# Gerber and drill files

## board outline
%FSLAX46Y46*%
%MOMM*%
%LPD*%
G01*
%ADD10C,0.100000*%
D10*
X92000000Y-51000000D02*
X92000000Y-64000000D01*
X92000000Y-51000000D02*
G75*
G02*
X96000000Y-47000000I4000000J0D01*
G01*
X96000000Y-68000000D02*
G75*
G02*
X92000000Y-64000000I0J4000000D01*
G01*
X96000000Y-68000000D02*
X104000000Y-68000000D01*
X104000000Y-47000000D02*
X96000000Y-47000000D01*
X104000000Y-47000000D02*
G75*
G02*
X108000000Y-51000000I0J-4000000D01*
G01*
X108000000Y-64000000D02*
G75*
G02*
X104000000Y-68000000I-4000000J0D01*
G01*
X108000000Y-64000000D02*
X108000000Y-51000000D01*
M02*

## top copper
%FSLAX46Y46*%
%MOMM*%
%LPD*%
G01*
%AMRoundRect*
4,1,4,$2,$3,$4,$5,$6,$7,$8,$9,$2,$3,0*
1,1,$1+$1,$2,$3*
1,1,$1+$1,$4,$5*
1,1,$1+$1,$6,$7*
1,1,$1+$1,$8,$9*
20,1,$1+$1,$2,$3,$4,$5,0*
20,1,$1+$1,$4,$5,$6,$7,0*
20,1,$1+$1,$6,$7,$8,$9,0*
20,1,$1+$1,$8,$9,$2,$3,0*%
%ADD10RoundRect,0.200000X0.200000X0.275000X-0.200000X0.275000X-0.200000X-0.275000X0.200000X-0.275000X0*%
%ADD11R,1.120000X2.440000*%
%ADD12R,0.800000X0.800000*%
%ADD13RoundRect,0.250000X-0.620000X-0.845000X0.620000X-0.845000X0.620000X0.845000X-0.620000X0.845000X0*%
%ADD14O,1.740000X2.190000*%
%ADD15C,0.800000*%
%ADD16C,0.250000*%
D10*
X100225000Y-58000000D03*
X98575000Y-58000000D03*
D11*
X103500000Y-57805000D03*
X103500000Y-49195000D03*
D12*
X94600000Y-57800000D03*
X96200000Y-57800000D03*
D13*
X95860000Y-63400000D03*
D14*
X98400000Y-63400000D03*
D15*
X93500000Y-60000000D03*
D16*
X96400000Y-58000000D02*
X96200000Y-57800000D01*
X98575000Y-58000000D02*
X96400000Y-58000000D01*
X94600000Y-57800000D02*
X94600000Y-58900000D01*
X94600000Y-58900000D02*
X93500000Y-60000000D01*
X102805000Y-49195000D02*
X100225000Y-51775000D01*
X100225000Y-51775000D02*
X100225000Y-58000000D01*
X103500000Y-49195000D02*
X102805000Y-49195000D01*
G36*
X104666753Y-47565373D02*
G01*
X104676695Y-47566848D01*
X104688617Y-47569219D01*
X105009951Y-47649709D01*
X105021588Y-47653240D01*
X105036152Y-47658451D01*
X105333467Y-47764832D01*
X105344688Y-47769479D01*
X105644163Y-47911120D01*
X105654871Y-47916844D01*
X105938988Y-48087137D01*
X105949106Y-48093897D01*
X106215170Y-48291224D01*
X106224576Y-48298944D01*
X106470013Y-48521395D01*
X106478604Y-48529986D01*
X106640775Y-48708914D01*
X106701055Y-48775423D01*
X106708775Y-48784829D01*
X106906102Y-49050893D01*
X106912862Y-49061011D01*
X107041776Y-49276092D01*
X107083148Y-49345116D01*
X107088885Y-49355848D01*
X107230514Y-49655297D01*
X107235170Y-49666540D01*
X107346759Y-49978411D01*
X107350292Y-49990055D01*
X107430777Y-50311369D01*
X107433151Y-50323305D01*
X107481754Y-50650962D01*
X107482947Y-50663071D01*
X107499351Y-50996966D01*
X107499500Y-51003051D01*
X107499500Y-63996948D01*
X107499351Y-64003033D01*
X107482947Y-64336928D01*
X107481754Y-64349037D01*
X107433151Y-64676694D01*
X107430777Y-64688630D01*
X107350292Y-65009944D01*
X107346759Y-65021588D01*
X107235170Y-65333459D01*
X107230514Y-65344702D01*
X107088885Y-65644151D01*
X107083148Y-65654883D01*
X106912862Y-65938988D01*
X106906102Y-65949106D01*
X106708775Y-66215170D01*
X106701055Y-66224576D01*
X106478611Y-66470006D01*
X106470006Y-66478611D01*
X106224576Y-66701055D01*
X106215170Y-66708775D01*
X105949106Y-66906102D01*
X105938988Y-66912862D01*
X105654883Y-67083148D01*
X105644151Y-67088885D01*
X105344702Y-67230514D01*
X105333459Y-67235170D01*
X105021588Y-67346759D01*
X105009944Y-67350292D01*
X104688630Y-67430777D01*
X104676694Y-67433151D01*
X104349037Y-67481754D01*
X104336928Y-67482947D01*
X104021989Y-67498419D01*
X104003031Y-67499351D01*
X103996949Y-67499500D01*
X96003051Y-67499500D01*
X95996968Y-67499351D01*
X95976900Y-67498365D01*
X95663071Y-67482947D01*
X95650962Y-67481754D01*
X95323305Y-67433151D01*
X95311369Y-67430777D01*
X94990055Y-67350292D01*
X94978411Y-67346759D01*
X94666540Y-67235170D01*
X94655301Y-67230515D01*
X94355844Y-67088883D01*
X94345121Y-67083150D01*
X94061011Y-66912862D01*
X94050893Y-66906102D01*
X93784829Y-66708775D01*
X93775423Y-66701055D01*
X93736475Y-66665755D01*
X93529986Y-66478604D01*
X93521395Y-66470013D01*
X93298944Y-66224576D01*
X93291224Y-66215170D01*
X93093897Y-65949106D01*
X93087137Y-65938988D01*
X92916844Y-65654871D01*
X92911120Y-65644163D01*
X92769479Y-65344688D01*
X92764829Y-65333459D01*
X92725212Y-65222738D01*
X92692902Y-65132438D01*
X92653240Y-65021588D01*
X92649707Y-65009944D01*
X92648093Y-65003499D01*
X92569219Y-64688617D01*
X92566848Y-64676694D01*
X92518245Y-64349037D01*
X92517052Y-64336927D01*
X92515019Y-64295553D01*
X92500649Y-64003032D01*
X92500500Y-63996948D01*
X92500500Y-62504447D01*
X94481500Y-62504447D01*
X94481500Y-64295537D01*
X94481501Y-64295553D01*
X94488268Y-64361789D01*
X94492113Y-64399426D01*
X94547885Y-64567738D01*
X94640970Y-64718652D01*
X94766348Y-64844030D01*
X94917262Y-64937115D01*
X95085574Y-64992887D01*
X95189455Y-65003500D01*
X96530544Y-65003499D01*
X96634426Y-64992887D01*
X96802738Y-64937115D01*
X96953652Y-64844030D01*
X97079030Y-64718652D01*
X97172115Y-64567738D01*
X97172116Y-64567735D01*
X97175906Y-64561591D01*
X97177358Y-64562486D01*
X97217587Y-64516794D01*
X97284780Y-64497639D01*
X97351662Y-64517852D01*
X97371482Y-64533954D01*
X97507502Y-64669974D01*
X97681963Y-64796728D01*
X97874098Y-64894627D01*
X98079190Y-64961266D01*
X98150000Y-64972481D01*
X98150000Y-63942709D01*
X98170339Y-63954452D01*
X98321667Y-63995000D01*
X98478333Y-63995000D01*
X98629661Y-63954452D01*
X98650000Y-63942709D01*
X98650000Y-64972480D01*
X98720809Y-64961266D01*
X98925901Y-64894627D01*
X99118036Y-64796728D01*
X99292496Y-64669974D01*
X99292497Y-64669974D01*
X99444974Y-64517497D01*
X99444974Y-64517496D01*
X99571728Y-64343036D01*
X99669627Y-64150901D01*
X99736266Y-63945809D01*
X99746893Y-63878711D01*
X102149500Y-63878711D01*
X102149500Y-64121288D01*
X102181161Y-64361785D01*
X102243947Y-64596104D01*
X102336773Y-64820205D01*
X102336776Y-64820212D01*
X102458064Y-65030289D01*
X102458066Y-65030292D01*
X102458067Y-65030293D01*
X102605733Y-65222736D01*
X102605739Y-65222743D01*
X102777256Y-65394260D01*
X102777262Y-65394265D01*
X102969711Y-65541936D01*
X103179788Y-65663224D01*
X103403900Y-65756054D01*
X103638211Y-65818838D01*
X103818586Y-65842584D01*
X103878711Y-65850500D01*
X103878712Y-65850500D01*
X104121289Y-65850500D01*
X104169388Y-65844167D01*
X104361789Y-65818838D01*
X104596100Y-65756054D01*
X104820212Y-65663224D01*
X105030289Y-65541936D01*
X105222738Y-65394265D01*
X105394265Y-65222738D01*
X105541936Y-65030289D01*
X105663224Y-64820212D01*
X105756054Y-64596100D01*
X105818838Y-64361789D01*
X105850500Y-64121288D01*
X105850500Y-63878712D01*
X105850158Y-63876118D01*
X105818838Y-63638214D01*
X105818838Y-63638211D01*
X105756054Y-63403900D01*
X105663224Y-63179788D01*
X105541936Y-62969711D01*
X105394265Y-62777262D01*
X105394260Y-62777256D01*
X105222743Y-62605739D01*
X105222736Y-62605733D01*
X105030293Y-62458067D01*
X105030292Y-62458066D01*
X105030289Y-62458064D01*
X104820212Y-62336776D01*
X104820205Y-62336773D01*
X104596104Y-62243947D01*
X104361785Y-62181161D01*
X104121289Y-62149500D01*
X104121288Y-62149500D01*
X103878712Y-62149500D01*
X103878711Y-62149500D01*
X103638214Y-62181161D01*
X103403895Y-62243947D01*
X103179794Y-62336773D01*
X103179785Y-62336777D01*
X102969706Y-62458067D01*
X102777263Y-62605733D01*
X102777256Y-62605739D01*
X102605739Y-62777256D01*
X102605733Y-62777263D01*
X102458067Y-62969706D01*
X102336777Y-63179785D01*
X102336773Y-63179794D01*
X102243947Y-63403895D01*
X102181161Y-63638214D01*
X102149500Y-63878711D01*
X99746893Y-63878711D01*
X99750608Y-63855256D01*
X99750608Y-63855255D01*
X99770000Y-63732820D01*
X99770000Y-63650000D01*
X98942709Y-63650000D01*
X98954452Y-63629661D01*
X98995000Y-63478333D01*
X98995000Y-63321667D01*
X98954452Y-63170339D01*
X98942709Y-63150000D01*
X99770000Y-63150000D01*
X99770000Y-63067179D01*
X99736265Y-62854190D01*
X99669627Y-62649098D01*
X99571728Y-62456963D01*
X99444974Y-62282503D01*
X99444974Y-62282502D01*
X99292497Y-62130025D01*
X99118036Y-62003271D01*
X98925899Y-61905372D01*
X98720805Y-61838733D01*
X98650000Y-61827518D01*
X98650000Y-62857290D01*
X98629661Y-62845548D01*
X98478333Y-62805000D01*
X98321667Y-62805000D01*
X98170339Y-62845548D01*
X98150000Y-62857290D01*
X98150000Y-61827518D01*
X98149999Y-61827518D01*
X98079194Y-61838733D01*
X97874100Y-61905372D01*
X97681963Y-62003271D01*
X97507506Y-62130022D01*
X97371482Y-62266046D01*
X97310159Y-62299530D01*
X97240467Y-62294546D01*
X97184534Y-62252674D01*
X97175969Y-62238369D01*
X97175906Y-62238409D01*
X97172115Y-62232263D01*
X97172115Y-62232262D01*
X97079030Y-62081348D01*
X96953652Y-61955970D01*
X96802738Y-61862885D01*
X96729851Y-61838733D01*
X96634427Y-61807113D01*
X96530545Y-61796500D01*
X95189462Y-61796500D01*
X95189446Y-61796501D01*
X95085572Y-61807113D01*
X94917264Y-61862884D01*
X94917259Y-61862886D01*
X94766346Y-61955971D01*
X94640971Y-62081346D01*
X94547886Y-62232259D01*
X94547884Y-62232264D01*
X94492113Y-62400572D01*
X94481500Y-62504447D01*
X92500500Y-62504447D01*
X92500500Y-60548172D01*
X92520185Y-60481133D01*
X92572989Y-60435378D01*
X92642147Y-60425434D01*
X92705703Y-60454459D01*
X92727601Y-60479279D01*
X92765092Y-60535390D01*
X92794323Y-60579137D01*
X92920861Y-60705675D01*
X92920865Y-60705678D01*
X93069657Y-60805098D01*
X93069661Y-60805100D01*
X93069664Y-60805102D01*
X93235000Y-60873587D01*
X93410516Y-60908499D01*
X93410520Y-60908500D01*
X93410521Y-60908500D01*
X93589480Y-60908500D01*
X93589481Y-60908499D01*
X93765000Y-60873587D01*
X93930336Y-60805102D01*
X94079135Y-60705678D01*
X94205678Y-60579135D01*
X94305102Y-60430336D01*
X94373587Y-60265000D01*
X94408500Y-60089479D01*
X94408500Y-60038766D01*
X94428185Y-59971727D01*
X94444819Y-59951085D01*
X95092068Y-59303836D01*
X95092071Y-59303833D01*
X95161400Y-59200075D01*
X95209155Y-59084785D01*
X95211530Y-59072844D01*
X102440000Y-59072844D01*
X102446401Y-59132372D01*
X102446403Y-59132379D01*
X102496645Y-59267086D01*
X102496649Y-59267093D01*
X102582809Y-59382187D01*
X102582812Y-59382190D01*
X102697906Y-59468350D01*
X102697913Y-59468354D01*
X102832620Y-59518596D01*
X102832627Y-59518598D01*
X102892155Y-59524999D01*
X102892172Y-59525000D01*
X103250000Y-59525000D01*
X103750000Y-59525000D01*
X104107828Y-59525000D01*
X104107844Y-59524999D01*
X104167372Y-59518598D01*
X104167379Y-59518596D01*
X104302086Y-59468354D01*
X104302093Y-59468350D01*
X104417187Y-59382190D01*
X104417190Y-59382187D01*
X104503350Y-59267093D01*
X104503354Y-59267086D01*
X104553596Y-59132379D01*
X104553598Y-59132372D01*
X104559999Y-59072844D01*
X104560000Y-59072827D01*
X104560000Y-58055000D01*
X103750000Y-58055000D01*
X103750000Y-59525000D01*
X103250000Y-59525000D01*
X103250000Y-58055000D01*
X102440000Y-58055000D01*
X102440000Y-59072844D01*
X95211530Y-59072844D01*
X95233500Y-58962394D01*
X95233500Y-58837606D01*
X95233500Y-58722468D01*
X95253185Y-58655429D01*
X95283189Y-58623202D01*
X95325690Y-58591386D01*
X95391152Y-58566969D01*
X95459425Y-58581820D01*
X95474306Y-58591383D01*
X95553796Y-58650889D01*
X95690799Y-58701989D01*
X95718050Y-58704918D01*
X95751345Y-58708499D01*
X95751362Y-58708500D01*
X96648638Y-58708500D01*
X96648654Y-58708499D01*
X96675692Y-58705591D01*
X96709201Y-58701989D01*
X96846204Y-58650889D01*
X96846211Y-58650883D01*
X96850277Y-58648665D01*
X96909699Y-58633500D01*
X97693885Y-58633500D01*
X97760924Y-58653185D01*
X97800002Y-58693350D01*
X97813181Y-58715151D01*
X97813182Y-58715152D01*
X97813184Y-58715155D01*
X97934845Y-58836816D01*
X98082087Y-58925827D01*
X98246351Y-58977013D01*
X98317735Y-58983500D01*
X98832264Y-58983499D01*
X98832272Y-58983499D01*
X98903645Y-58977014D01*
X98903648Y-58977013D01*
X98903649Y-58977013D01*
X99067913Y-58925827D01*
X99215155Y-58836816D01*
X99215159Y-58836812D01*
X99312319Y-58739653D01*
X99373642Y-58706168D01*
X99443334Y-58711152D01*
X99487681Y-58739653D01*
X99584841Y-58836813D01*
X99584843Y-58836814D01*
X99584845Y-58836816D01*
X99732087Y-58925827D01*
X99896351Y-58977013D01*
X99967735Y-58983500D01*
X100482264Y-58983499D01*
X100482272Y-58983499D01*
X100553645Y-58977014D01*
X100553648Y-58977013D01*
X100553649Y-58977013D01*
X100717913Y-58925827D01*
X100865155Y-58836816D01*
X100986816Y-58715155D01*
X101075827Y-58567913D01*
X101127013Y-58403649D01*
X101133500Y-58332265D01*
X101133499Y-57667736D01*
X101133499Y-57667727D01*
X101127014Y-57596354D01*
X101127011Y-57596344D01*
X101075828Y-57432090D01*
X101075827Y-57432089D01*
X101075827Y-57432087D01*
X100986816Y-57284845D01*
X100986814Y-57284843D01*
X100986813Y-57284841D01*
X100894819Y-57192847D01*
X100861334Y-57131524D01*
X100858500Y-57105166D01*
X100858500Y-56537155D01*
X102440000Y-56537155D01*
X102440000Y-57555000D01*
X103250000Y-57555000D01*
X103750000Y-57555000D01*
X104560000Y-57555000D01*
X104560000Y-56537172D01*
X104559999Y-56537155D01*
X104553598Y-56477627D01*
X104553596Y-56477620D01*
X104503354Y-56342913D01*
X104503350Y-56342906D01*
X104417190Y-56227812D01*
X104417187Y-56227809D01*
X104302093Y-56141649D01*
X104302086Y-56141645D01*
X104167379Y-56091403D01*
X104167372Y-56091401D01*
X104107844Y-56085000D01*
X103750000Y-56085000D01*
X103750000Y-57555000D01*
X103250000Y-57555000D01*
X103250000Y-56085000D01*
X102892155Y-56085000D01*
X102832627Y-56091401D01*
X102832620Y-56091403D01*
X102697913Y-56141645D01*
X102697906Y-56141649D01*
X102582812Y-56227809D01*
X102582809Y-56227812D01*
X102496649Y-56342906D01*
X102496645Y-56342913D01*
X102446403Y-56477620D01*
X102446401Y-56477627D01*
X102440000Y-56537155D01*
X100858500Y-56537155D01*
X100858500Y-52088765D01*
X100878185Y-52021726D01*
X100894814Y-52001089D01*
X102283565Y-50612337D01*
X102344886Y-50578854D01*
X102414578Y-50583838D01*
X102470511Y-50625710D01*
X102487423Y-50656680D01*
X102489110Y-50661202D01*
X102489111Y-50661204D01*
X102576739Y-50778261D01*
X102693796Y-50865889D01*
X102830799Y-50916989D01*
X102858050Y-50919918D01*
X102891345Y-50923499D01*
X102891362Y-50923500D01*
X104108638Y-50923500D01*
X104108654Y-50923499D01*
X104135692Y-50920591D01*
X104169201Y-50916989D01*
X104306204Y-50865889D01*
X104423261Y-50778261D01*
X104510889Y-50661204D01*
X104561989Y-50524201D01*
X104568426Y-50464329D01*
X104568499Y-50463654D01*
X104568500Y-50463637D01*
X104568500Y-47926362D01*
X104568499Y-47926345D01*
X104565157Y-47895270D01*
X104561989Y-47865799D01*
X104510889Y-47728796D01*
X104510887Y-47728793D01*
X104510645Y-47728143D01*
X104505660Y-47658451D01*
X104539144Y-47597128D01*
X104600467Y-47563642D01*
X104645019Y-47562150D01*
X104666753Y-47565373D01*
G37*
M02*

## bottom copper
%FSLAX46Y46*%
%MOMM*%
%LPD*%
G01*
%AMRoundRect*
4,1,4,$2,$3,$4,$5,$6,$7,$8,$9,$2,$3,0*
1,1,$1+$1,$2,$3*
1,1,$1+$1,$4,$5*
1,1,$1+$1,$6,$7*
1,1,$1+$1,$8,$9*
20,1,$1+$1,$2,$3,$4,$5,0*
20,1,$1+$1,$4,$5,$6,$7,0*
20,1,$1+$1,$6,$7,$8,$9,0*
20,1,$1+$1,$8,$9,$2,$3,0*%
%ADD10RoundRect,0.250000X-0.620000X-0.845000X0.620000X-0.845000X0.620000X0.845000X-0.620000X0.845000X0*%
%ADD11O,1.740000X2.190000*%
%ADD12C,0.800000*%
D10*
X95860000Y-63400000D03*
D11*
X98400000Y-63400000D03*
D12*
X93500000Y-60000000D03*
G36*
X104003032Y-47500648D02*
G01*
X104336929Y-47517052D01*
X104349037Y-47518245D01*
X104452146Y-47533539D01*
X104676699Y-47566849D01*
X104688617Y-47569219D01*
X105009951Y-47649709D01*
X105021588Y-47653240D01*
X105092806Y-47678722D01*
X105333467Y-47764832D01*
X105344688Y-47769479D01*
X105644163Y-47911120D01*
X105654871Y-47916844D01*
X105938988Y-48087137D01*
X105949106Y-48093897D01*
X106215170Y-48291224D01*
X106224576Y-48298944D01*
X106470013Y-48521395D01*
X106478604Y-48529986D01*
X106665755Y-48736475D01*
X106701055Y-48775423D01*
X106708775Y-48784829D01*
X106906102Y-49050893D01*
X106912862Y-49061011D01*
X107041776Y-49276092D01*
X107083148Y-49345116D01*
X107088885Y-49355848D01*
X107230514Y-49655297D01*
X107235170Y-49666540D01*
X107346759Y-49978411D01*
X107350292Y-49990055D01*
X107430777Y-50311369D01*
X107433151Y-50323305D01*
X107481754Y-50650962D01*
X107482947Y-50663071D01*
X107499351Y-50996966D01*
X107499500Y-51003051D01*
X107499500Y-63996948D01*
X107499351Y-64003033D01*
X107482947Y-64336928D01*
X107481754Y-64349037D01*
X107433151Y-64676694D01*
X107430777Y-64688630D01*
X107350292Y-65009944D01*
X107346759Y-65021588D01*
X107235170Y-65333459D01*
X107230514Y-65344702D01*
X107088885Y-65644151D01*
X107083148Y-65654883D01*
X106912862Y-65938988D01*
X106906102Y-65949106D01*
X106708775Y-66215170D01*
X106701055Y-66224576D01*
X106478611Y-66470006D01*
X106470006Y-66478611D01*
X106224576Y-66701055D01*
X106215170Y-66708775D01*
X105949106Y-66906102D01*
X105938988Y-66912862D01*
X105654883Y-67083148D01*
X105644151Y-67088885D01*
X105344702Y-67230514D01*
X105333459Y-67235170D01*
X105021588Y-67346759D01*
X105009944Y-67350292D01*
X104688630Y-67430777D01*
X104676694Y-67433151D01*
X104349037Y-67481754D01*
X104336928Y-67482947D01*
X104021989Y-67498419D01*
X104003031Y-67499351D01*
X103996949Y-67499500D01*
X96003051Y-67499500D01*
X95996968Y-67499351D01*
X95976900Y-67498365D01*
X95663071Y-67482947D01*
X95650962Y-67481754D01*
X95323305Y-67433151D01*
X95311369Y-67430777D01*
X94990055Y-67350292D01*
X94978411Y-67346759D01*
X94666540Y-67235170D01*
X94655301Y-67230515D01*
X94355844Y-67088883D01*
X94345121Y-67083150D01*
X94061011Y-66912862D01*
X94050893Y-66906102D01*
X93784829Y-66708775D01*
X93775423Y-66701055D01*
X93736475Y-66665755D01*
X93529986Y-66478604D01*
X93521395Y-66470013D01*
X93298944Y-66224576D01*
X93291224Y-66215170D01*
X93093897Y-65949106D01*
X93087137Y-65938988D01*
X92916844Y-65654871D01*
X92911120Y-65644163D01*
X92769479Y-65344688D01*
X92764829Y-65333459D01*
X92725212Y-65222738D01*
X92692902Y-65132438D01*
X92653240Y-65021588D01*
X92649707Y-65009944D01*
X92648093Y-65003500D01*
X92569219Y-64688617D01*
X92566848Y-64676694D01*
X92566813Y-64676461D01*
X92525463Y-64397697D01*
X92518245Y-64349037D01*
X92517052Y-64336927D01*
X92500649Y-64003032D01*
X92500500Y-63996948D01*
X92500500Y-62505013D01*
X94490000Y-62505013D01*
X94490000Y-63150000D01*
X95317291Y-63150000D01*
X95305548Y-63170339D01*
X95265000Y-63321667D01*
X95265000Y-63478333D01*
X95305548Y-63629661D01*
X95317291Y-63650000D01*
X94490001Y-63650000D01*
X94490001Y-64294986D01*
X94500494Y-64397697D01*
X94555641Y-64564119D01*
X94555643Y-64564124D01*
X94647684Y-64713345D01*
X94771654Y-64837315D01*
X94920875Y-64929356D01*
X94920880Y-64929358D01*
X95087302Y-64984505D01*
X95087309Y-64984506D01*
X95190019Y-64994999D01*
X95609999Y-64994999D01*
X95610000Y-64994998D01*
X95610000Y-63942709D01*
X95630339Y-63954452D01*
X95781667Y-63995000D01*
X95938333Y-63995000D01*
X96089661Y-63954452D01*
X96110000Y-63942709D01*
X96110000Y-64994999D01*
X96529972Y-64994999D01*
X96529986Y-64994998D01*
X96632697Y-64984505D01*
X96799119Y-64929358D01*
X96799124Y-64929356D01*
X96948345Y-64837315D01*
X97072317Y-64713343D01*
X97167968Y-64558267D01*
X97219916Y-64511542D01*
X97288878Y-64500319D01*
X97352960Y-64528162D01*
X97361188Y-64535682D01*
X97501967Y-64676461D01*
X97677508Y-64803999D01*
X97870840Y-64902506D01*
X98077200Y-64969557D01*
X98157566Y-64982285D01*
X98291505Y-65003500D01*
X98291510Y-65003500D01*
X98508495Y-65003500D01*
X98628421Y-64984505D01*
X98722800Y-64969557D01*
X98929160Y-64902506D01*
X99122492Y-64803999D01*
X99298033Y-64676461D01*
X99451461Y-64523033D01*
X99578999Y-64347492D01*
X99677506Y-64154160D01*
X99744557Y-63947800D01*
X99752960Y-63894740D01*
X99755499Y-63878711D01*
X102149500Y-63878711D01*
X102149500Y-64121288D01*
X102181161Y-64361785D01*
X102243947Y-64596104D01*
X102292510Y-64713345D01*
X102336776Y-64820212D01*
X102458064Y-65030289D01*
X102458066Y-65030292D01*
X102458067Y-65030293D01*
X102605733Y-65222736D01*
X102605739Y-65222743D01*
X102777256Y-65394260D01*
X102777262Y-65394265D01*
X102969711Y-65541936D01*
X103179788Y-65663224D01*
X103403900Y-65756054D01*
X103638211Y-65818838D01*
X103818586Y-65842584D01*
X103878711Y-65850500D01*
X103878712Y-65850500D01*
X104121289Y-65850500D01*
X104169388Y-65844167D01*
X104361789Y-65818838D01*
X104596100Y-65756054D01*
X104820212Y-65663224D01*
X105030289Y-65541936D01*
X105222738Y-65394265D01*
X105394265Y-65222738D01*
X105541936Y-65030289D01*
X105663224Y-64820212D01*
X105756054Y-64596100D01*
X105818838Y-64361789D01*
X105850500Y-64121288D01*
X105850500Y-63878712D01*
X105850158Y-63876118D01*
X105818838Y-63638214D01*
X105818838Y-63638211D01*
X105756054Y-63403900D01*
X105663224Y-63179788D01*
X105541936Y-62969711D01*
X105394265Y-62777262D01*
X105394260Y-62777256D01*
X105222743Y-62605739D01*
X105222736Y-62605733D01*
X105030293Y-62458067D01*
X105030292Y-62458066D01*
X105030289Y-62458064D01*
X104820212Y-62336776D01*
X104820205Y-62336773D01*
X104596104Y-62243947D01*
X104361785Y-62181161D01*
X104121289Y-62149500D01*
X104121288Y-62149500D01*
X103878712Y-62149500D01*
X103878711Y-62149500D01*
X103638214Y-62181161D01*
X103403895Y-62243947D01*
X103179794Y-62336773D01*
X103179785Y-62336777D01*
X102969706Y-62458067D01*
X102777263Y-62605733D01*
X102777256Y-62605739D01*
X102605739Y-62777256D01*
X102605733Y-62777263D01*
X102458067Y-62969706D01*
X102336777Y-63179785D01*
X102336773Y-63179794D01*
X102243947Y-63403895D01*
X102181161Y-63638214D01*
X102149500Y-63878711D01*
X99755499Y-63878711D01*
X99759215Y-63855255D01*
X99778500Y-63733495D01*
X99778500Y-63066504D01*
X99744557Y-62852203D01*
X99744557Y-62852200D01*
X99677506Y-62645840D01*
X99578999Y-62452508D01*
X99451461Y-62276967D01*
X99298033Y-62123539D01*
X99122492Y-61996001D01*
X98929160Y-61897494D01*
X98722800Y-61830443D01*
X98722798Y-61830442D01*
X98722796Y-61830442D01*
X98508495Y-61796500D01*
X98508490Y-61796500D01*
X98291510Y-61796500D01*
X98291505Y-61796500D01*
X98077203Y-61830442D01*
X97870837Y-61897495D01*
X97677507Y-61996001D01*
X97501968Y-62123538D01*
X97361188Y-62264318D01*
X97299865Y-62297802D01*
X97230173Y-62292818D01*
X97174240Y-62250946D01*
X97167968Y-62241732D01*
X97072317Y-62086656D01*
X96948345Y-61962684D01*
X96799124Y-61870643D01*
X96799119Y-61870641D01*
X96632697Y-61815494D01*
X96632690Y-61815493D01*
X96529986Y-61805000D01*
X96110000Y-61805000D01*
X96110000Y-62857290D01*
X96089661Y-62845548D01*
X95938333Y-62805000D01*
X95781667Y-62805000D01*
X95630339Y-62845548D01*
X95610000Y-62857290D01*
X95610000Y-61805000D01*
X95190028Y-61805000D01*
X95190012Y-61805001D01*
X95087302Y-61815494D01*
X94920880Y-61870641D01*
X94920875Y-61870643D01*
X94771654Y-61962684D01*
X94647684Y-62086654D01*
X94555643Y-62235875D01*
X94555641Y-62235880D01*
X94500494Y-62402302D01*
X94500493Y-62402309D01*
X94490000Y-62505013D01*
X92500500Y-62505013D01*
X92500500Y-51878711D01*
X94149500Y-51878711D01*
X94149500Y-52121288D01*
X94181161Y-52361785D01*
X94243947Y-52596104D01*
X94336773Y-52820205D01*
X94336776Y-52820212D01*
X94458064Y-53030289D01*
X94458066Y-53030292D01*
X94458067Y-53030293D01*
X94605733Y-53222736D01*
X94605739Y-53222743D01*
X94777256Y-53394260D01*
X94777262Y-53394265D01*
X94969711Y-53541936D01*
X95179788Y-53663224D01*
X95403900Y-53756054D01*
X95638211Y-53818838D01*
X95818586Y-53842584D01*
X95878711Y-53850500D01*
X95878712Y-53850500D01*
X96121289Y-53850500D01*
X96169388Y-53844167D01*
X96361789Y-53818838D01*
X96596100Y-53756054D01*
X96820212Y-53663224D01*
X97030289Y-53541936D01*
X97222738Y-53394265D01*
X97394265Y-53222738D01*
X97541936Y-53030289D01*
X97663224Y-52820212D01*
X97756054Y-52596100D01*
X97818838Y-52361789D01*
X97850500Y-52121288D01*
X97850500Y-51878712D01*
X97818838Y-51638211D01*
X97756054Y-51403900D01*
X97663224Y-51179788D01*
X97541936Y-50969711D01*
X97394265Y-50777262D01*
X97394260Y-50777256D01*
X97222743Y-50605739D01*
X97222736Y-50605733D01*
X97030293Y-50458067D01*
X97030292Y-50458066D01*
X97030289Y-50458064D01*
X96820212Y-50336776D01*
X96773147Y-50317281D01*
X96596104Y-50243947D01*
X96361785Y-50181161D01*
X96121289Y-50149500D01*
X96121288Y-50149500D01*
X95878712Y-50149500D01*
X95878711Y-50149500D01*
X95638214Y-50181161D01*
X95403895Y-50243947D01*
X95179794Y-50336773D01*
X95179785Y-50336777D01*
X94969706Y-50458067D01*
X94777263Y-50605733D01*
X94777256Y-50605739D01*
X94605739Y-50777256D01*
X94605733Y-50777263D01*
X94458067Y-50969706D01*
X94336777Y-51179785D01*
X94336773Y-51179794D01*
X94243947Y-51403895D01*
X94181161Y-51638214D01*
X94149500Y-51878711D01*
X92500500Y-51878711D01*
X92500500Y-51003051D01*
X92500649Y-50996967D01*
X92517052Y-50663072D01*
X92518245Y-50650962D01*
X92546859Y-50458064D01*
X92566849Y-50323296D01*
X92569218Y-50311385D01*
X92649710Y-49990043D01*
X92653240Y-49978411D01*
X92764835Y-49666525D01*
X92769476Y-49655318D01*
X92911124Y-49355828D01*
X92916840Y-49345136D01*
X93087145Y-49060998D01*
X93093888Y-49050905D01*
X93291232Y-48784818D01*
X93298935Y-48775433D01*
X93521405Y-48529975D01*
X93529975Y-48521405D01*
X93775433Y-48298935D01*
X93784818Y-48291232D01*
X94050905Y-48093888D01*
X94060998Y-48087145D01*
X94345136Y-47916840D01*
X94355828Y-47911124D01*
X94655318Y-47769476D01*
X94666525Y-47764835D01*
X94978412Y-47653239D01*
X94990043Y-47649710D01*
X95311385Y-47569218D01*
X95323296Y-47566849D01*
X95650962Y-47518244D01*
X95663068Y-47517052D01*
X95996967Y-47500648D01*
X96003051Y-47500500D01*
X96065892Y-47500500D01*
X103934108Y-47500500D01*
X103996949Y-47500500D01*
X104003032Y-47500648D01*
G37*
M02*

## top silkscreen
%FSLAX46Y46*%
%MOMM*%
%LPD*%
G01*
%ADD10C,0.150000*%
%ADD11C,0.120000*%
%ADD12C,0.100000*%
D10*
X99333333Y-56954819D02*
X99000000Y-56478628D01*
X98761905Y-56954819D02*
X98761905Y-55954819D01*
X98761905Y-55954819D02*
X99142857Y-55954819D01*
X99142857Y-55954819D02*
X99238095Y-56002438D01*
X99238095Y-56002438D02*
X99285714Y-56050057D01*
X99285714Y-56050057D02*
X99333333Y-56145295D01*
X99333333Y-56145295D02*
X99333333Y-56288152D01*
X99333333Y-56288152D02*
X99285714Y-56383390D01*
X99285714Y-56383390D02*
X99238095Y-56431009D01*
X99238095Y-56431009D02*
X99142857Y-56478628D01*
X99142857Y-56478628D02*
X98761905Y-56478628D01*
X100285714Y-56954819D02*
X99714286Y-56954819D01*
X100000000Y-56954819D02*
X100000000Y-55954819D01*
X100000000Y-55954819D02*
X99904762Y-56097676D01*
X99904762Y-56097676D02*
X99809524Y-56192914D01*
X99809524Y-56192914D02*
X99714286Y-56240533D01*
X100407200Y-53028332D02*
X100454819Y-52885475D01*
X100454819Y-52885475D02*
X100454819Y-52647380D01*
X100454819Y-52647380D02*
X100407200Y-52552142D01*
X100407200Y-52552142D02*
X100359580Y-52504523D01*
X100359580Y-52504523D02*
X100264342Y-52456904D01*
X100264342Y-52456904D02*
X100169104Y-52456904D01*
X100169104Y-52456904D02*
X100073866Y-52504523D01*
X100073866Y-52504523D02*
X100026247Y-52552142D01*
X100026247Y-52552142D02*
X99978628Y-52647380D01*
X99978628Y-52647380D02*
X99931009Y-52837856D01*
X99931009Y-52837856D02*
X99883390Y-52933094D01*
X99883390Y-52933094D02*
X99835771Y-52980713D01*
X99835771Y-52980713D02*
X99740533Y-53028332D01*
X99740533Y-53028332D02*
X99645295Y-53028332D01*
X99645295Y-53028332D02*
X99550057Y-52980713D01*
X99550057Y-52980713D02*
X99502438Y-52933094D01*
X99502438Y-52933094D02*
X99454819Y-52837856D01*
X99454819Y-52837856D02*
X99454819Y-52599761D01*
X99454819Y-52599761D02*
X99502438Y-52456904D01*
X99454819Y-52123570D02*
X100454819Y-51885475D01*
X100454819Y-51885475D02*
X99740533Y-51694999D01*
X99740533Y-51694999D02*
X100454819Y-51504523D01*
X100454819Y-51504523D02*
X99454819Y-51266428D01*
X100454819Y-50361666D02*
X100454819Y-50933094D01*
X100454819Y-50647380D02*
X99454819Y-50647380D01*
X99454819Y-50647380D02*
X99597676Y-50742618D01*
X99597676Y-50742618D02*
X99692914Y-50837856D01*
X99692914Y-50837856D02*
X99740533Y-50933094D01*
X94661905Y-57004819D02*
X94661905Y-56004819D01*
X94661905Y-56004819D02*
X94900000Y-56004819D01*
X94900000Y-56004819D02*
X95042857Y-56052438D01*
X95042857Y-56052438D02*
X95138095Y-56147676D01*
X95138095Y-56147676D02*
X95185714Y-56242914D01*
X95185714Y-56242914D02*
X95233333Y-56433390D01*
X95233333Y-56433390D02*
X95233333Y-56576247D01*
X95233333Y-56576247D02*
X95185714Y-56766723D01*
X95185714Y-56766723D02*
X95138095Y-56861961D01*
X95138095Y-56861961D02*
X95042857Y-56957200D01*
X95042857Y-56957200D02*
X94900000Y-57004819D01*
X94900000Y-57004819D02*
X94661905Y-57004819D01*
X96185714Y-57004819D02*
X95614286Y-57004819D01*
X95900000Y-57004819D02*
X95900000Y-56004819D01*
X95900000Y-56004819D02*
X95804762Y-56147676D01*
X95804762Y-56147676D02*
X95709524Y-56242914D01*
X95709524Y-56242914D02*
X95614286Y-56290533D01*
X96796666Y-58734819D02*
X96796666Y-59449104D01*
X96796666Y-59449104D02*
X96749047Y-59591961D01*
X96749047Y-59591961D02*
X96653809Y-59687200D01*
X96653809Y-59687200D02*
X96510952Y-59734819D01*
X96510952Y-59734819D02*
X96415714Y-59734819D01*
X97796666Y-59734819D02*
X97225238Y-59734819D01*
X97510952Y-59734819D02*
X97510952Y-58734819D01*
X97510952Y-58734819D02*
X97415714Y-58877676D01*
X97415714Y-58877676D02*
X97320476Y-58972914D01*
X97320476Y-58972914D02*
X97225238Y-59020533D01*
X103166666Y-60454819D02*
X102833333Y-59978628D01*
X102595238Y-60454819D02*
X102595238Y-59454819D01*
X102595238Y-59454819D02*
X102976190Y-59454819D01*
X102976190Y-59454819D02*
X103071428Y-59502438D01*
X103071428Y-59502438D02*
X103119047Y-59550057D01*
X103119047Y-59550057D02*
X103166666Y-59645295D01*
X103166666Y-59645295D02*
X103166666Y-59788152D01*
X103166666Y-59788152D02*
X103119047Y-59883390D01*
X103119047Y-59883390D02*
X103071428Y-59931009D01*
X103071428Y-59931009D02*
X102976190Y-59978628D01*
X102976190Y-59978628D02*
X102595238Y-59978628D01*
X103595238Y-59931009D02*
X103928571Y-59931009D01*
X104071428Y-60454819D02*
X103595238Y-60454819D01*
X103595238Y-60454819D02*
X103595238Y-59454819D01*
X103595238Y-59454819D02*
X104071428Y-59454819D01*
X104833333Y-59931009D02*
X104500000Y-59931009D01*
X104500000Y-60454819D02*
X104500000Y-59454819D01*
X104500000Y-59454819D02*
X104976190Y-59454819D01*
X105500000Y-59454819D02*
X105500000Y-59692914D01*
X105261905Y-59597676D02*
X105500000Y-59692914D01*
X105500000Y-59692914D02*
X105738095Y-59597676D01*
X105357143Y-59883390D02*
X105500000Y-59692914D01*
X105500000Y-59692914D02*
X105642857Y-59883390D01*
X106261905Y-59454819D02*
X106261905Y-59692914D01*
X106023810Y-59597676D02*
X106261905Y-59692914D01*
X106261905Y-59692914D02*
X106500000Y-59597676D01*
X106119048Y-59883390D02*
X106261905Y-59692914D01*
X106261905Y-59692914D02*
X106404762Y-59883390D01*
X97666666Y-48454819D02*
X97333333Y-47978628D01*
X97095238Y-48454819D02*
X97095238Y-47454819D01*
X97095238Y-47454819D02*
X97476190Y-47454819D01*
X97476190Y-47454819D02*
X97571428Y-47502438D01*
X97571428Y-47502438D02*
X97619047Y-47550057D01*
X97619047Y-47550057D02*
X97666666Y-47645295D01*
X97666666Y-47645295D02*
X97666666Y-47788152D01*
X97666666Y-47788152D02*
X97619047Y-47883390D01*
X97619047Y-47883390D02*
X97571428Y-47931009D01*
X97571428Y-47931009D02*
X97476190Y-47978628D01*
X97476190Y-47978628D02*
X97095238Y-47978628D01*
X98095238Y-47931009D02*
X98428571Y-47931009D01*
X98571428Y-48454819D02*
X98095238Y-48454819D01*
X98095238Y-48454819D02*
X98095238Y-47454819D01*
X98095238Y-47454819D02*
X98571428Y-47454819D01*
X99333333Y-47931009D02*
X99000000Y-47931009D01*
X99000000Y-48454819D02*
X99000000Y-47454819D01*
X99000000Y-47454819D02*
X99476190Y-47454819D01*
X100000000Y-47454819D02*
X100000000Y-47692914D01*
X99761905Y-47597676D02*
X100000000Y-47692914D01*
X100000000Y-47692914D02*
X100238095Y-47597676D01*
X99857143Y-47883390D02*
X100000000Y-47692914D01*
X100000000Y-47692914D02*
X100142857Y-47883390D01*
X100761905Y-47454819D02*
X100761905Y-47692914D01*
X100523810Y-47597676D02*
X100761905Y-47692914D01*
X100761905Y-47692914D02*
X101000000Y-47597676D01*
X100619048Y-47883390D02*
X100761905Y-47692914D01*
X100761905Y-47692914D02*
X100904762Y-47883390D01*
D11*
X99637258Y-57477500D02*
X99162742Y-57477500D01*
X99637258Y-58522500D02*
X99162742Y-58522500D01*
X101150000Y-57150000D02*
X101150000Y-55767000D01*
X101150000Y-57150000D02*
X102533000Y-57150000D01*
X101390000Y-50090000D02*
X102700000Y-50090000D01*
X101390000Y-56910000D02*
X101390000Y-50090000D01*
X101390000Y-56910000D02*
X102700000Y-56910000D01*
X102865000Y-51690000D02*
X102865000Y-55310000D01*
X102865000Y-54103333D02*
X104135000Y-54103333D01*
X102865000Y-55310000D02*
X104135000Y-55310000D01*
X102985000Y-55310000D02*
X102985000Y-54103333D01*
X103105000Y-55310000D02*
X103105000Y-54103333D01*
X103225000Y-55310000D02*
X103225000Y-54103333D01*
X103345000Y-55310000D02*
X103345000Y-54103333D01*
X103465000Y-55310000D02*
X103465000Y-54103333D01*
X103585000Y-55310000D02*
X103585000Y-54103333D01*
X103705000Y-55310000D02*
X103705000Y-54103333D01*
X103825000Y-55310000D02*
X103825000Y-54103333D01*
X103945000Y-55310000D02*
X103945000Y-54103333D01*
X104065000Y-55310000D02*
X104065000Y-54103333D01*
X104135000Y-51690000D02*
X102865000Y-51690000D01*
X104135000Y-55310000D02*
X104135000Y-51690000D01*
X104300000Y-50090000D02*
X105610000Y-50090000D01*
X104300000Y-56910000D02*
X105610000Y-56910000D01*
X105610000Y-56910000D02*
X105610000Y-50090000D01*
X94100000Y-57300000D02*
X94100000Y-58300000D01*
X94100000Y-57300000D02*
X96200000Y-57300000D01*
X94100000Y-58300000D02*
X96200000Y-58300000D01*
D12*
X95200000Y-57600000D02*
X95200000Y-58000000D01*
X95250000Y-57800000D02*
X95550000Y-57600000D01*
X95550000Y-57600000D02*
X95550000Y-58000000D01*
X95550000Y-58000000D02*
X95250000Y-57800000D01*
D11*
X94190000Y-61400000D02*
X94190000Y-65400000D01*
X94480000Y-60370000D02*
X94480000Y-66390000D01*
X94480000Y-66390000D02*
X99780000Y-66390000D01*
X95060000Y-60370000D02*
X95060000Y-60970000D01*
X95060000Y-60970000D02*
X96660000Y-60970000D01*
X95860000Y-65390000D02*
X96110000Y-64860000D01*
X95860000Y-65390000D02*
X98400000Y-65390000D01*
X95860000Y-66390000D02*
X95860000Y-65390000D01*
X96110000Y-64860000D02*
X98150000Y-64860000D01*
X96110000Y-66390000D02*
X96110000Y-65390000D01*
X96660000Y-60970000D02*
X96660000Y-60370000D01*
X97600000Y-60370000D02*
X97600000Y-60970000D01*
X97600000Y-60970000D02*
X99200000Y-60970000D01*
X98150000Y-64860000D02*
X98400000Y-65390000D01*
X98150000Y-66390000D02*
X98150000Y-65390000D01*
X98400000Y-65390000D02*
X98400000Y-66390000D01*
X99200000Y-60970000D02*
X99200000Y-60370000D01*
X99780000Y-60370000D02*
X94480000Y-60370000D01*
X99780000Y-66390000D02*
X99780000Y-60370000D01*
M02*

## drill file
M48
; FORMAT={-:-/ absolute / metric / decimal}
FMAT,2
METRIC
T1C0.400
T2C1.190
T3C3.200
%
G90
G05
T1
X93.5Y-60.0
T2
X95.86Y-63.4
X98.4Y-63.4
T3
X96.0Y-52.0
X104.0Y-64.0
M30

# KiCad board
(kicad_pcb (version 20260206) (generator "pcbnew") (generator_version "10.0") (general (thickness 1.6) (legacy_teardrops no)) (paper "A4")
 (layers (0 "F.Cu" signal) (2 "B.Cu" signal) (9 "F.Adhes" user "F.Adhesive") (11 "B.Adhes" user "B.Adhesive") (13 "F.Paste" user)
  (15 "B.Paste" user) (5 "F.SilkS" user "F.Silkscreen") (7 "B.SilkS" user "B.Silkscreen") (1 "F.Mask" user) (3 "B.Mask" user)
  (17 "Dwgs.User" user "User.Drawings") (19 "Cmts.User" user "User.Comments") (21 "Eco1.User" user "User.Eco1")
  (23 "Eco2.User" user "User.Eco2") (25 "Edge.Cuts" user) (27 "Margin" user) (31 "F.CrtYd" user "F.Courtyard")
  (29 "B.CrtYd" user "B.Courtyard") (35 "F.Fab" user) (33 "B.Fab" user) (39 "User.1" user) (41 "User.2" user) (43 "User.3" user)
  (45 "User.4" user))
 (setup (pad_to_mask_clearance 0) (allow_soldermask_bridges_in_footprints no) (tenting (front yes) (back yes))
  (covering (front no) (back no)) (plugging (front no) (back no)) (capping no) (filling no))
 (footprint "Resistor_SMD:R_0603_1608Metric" (layer "F.Cu") (at 99.4 58 180)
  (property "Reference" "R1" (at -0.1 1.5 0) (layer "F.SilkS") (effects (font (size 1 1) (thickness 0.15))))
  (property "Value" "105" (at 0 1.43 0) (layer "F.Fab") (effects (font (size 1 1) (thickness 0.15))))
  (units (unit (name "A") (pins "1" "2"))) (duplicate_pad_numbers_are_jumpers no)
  (fp_line (start -0.237258 0.5225) (end 0.237258 0.5225) (stroke (width 0.12) (type solid)) (layer "F.SilkS"))
  (fp_line (start -0.237258 -0.5225) (end 0.237258 -0.5225) (stroke (width 0.12) (type solid)) (layer "F.SilkS"))
  (pad "1" smd roundrect (at -0.825 0 180) (size 0.8 0.95) (layers "F.Cu" "F.Mask" "F.Paste") (roundrect_rratio 0.25) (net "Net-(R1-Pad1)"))
  (pad "2" smd roundrect (at 0.825 0 180) (size 0.8 0.95) (layers "F.Cu" "F.Mask" "F.Paste") (roundrect_rratio 0.25) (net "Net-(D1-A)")))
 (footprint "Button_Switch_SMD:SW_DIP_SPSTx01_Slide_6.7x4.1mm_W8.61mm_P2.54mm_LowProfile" (layer "F.Cu") (at 103.5 53.5 90)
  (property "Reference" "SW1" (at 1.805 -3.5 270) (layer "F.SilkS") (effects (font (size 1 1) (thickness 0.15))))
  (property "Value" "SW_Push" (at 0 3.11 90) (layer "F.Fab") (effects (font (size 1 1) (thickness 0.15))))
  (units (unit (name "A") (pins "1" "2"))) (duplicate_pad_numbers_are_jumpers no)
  (fp_line (start -3.65 -2.35) (end -2.267 -2.35) (stroke (width 0.12) (type solid)) (layer "F.SilkS"))
  (fp_line (start -3.65 -2.35) (end -3.65 -0.967) (stroke (width 0.12) (type solid)) (layer "F.SilkS"))
  (fp_line (start 3.41 -2.11) (end 3.41 -0.8) (stroke (width 0.12) (type solid)) (layer "F.SilkS"))
  (fp_line (start -3.41 -2.11) (end 3.41 -2.11) (stroke (width 0.12) (type solid)) (layer "F.SilkS"))
  (fp_line (start -3.41 -2.11) (end -3.41 -0.8) (stroke (width 0.12) (type solid)) (layer "F.SilkS"))
  (fp_line (start 1.81 -0.635) (end -1.81 -0.635) (stroke (width 0.12) (type solid)) (layer "F.SilkS"))
  (fp_line (start -0.603333 -0.635) (end -0.603333 0.635) (stroke (width 0.12) (type solid)) (layer "F.SilkS"))
  (fp_line (start -1.81 -0.635) (end -1.81 0.635) (stroke (width 0.12) (type solid)) (layer "F.SilkS"))
  (fp_line (start -1.81 -0.515) (end -0.603333 -0.515) (stroke (width 0.12) (type solid)) (layer "F.SilkS"))
  (fp_line (start -1.81 -0.395) (end -0.603333 -0.395) (stroke (width 0.12) (type solid)) (layer "F.SilkS"))
  (fp_line (start -1.81 -0.275) (end -0.603333 -0.275) (stroke (width 0.12) (type solid)) (layer "F.SilkS"))
  (fp_line (start -1.81 -0.155) (end -0.603333 -0.155) (stroke (width 0.12) (type solid)) (layer "F.SilkS"))
  (fp_line (start -1.81 -0.035) (end -0.603333 -0.035) (stroke (width 0.12) (type solid)) (layer "F.SilkS"))
  (fp_line (start -1.81 0.085) (end -0.603333 0.085) (stroke (width 0.12) (type solid)) (layer "F.SilkS"))
  (fp_line (start -1.81 0.205) (end -0.603333 0.205) (stroke (width 0.12) (type solid)) (layer "F.SilkS"))
  (fp_line (start -1.81 0.325) (end -0.603333 0.325) (stroke (width 0.12) (type solid)) (layer "F.SilkS"))
  (fp_line (start -1.81 0.445) (end -0.603333 0.445) (stroke (width 0.12) (type solid)) (layer "F.SilkS"))
  (fp_line (start -1.81 0.565) (end -0.603333 0.565) (stroke (width 0.12) (type solid)) (layer "F.SilkS"))
  (fp_line (start 1.81 0.635) (end 1.81 -0.635) (stroke (width 0.12) (type solid)) (layer "F.SilkS"))
  (fp_line (start -1.81 0.635) (end 1.81 0.635) (stroke (width 0.12) (type solid)) (layer "F.SilkS"))
  (fp_line (start 3.41 0.8) (end 3.41 2.11) (stroke (width 0.12) (type solid)) (layer "F.SilkS"))
  (fp_line (start -3.41 0.8) (end -3.41 2.11) (stroke (width 0.12) (type solid)) (layer "F.SilkS"))
  (fp_line (start -3.41 2.11) (end 3.41 2.11) (stroke (width 0.12) (type solid)) (layer "F.SilkS"))
  (pad "1" smd rect (at -4.305 0 90) (size 2.44 1.12) (layers "F.Cu" "F.Mask" "F.Paste") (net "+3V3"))
  (pad "2" smd rect (at 4.305 0 90) (size 2.44 1.12) (layers "F.Cu" "F.Mask" "F.Paste") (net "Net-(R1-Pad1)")))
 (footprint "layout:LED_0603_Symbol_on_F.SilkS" (layer "F.Cu") (at 95.4 57.8)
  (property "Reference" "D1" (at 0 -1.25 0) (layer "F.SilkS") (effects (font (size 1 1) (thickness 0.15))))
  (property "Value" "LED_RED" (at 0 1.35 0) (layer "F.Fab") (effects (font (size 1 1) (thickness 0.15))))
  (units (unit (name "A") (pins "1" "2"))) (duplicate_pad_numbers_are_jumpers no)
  (fp_line (start -1.3 -0.5) (end -1.3 0.5) (stroke (width 0.12) (type solid)) (layer "F.SilkS"))
  (fp_line (start -1.3 -0.5) (end 0.8 -0.5) (stroke (width 0.12) (type solid)) (layer "F.SilkS"))
  (fp_line (start -1.3 0.5) (end 0.8 0.5) (stroke (width 0.12) (type solid)) (layer "F.SilkS"))
  (fp_line (start -0.2 -0.2) (end -0.2 0.2) (stroke (width 0.1) (type solid)) (layer "F.SilkS"))
  (fp_line (start -0.15 0) (end 0.15 -0.2) (stroke (width 0.1) (type solid)) (layer "F.SilkS"))
  (fp_line (start 0.15 -0.2) (end 0.15 0.2) (stroke (width 0.1) (type solid)) (layer "F.SilkS"))
  (fp_line (start 0.15 0.2) (end -0.15 0) (stroke (width 0.1) (type solid)) (layer "F.SilkS"))
  (pad "1" smd rect (at -0.8 0 180) (size 0.8 0.8) (layers "F.Cu" "F.Mask" "F.Paste") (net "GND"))
  (pad "2" smd rect (at 0.8 0 180) (size 0.8 0.8) (layers "F.Cu" "F.Mask" "F.Paste") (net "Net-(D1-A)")))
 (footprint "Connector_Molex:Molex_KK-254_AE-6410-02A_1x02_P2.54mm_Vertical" (layer "F.Cu") (at 95.86 63.4)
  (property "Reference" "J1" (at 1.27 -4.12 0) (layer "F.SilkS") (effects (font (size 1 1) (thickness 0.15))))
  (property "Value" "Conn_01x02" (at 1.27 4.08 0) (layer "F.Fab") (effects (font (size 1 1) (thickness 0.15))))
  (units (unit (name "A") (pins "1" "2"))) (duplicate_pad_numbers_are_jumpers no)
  (fp_line (start -1.67 -2) (end -1.67 2) (stroke (width 0.12) (type solid)) (layer "F.SilkS"))
  (fp_line (start -1.38 -3.03) (end -1.38 2.99) (stroke (width 0.12) (type solid)) (layer "F.SilkS"))
  (fp_line (start -1.38 2.99) (end 3.92 2.99) (stroke (width 0.12) (type solid)) (layer "F.SilkS"))
  (fp_line (start -0.8 -3.03) (end -0.8 -2.43) (stroke (width 0.12) (type solid)) (layer "F.SilkS"))
  (fp_line (start -0.8 -2.43) (end 0.8 -2.43) (stroke (width 0.12) (type solid)) (layer "F.SilkS"))
  (fp_line (start 0 1.99) (end 0.25 1.46) (stroke (width 0.12) (type solid)) (layer "F.SilkS"))
  (fp_line (start 0 1.99) (end 2.54 1.99) (stroke (width 0.12) (type solid)) (layer "F.SilkS"))
  (fp_line (start 0 2.99) (end 0 1.99) (stroke (width 0.12) (type solid)) (layer "F.SilkS"))
  (fp_line (start 0.25 1.46) (end 2.29 1.46) (stroke (width 0.12) (type solid)) (layer "F.SilkS"))
  (fp_line (start 0.25 2.99) (end 0.25 1.99) (stroke (width 0.12) (type solid)) (layer "F.SilkS"))
  (fp_line (start 0.8 -2.43) (end 0.8 -3.03) (stroke (width 0.12) (type solid)) (layer "F.SilkS"))
  (fp_line (start 1.74 -3.03) (end 1.74 -2.43) (stroke (width 0.12) (type solid)) (layer "F.SilkS"))
  (fp_line (start 1.74 -2.43) (end 3.34 -2.43) (stroke (width 0.12) (type solid)) (layer "F.SilkS"))
  (fp_line (start 2.29 1.46) (end 2.54 1.99) (stroke (width 0.12) (type solid)) (layer "F.SilkS"))
  (fp_line (start 2.29 2.99) (end 2.29 1.99) (stroke (width 0.12) (type solid)) (layer "F.SilkS"))
  (fp_line (start 2.54 1.99) (end 2.54 2.99) (stroke (width 0.12) (type solid)) (layer "F.SilkS"))
  (fp_line (start 3.34 -2.43) (end 3.34 -3.03) (stroke (width 0.12) (type solid)) (layer "F.SilkS"))
  (fp_line (start 3.92 -3.03) (end -1.38 -3.03) (stroke (width 0.12) (type solid)) (layer "F.SilkS"))
  (fp_line (start 3.92 2.99) (end 3.92 -3.03) (stroke (width 0.12) (type solid)) (layer "F.SilkS"))
  (pad "1" thru_hole roundrect (at 0 0) (size 1.74 2.19) (drill 1.19) (layers "*.Cu" "*.Mask") (remove_unused_layers no)
   (roundrect_rratio 0.143678) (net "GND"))
  (pad "2" thru_hole oval (at 2.54 0) (size 1.74 2.19) (drill 1.19) (layers "*.Cu" "*.Mask") (remove_unused_layers no) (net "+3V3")))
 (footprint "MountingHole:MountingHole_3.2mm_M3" (layer "F.Cu") (at 104 64)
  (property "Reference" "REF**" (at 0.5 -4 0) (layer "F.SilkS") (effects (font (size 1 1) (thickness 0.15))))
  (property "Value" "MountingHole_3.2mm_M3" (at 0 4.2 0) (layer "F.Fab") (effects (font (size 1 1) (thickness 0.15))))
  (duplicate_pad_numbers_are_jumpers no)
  (pad "" np_thru_hole circle (at 0 0) (size 3.2 3.2) (drill 3.2) (layers "*.Cu" "*.Mask")))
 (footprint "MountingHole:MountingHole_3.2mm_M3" (layer "F.Cu") (at 96 52)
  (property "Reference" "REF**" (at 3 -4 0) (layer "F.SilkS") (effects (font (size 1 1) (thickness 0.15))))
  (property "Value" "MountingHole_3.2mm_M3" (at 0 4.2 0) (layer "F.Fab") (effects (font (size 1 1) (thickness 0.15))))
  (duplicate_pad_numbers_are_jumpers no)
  (pad "" np_thru_hole circle (at 0 0) (size 3.2 3.2) (drill 3.2) (layers "*.Cu" "*.Mask")))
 (gr_line (start 92 51) (end 92 64) (stroke (width 0.1) (type default)) (layer "Edge.Cuts"))
 (gr_arc (start 92 51) (mid 93.171573 48.171573) (end 96 47) (stroke (width 0.1) (type default)) (layer "Edge.Cuts"))
 (gr_arc (start 96 68) (mid 93.171573 66.828427) (end 92 64) (stroke (width 0.1) (type default)) (layer "Edge.Cuts"))
 (gr_line (start 96 68) (end 104 68) (stroke (width 0.1) (type default)) (layer "Edge.Cuts"))
 (gr_line (start 104 47) (end 96 47) (stroke (width 0.1) (type default)) (layer "Edge.Cuts"))
 (gr_arc (start 104 47) (mid 106.828427 48.171573) (end 108 51) (stroke (width 0.1) (type default)) (layer "Edge.Cuts"))
 (gr_arc (start 108 64) (mid 106.828427 66.828427) (end 104 68) (stroke (width 0.1) (type default)) (layer "Edge.Cuts"))
 (gr_line (start 108 64) (end 108 51) (stroke (width 0.1) (type default)) (layer "Edge.Cuts"))
 (segment (start 96.4 58) (end 96.2 57.8) (width 0.25) (layer "F.Cu") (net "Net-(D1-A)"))
 (segment (start 98.575 58) (end 96.4 58) (width 0.25) (layer "F.Cu") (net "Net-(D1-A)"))
 (segment (start 94.6 57.8) (end 94.6 58.9) (width 0.25) (layer "F.Cu") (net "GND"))
 (segment (start 94.6 58.9) (end 93.5 60) (width 0.25) (layer "F.Cu") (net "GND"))
 (via (at 93.5 60) (size 0.8) (drill 0.4) (layers "F.Cu" "B.Cu") (free yes) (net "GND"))
 (segment (start 102.805 49.195) (end 100.225 51.775) (width 0.25) (layer "F.Cu") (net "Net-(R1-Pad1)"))
 (segment (start 100.225 51.775) (end 100.225 58) (width 0.25) (layer "F.Cu") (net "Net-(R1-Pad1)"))
 (segment (start 103.5 49.195) (end 102.805 49.195) (width 0.25) (layer "F.Cu") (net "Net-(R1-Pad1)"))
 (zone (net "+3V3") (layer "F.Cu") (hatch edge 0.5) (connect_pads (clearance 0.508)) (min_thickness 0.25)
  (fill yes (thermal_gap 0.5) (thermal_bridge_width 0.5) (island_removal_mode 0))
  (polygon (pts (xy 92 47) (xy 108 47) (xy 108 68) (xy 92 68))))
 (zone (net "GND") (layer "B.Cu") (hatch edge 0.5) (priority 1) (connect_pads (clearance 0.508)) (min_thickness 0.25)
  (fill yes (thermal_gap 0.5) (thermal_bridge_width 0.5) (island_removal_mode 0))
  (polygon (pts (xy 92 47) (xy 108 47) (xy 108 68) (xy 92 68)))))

